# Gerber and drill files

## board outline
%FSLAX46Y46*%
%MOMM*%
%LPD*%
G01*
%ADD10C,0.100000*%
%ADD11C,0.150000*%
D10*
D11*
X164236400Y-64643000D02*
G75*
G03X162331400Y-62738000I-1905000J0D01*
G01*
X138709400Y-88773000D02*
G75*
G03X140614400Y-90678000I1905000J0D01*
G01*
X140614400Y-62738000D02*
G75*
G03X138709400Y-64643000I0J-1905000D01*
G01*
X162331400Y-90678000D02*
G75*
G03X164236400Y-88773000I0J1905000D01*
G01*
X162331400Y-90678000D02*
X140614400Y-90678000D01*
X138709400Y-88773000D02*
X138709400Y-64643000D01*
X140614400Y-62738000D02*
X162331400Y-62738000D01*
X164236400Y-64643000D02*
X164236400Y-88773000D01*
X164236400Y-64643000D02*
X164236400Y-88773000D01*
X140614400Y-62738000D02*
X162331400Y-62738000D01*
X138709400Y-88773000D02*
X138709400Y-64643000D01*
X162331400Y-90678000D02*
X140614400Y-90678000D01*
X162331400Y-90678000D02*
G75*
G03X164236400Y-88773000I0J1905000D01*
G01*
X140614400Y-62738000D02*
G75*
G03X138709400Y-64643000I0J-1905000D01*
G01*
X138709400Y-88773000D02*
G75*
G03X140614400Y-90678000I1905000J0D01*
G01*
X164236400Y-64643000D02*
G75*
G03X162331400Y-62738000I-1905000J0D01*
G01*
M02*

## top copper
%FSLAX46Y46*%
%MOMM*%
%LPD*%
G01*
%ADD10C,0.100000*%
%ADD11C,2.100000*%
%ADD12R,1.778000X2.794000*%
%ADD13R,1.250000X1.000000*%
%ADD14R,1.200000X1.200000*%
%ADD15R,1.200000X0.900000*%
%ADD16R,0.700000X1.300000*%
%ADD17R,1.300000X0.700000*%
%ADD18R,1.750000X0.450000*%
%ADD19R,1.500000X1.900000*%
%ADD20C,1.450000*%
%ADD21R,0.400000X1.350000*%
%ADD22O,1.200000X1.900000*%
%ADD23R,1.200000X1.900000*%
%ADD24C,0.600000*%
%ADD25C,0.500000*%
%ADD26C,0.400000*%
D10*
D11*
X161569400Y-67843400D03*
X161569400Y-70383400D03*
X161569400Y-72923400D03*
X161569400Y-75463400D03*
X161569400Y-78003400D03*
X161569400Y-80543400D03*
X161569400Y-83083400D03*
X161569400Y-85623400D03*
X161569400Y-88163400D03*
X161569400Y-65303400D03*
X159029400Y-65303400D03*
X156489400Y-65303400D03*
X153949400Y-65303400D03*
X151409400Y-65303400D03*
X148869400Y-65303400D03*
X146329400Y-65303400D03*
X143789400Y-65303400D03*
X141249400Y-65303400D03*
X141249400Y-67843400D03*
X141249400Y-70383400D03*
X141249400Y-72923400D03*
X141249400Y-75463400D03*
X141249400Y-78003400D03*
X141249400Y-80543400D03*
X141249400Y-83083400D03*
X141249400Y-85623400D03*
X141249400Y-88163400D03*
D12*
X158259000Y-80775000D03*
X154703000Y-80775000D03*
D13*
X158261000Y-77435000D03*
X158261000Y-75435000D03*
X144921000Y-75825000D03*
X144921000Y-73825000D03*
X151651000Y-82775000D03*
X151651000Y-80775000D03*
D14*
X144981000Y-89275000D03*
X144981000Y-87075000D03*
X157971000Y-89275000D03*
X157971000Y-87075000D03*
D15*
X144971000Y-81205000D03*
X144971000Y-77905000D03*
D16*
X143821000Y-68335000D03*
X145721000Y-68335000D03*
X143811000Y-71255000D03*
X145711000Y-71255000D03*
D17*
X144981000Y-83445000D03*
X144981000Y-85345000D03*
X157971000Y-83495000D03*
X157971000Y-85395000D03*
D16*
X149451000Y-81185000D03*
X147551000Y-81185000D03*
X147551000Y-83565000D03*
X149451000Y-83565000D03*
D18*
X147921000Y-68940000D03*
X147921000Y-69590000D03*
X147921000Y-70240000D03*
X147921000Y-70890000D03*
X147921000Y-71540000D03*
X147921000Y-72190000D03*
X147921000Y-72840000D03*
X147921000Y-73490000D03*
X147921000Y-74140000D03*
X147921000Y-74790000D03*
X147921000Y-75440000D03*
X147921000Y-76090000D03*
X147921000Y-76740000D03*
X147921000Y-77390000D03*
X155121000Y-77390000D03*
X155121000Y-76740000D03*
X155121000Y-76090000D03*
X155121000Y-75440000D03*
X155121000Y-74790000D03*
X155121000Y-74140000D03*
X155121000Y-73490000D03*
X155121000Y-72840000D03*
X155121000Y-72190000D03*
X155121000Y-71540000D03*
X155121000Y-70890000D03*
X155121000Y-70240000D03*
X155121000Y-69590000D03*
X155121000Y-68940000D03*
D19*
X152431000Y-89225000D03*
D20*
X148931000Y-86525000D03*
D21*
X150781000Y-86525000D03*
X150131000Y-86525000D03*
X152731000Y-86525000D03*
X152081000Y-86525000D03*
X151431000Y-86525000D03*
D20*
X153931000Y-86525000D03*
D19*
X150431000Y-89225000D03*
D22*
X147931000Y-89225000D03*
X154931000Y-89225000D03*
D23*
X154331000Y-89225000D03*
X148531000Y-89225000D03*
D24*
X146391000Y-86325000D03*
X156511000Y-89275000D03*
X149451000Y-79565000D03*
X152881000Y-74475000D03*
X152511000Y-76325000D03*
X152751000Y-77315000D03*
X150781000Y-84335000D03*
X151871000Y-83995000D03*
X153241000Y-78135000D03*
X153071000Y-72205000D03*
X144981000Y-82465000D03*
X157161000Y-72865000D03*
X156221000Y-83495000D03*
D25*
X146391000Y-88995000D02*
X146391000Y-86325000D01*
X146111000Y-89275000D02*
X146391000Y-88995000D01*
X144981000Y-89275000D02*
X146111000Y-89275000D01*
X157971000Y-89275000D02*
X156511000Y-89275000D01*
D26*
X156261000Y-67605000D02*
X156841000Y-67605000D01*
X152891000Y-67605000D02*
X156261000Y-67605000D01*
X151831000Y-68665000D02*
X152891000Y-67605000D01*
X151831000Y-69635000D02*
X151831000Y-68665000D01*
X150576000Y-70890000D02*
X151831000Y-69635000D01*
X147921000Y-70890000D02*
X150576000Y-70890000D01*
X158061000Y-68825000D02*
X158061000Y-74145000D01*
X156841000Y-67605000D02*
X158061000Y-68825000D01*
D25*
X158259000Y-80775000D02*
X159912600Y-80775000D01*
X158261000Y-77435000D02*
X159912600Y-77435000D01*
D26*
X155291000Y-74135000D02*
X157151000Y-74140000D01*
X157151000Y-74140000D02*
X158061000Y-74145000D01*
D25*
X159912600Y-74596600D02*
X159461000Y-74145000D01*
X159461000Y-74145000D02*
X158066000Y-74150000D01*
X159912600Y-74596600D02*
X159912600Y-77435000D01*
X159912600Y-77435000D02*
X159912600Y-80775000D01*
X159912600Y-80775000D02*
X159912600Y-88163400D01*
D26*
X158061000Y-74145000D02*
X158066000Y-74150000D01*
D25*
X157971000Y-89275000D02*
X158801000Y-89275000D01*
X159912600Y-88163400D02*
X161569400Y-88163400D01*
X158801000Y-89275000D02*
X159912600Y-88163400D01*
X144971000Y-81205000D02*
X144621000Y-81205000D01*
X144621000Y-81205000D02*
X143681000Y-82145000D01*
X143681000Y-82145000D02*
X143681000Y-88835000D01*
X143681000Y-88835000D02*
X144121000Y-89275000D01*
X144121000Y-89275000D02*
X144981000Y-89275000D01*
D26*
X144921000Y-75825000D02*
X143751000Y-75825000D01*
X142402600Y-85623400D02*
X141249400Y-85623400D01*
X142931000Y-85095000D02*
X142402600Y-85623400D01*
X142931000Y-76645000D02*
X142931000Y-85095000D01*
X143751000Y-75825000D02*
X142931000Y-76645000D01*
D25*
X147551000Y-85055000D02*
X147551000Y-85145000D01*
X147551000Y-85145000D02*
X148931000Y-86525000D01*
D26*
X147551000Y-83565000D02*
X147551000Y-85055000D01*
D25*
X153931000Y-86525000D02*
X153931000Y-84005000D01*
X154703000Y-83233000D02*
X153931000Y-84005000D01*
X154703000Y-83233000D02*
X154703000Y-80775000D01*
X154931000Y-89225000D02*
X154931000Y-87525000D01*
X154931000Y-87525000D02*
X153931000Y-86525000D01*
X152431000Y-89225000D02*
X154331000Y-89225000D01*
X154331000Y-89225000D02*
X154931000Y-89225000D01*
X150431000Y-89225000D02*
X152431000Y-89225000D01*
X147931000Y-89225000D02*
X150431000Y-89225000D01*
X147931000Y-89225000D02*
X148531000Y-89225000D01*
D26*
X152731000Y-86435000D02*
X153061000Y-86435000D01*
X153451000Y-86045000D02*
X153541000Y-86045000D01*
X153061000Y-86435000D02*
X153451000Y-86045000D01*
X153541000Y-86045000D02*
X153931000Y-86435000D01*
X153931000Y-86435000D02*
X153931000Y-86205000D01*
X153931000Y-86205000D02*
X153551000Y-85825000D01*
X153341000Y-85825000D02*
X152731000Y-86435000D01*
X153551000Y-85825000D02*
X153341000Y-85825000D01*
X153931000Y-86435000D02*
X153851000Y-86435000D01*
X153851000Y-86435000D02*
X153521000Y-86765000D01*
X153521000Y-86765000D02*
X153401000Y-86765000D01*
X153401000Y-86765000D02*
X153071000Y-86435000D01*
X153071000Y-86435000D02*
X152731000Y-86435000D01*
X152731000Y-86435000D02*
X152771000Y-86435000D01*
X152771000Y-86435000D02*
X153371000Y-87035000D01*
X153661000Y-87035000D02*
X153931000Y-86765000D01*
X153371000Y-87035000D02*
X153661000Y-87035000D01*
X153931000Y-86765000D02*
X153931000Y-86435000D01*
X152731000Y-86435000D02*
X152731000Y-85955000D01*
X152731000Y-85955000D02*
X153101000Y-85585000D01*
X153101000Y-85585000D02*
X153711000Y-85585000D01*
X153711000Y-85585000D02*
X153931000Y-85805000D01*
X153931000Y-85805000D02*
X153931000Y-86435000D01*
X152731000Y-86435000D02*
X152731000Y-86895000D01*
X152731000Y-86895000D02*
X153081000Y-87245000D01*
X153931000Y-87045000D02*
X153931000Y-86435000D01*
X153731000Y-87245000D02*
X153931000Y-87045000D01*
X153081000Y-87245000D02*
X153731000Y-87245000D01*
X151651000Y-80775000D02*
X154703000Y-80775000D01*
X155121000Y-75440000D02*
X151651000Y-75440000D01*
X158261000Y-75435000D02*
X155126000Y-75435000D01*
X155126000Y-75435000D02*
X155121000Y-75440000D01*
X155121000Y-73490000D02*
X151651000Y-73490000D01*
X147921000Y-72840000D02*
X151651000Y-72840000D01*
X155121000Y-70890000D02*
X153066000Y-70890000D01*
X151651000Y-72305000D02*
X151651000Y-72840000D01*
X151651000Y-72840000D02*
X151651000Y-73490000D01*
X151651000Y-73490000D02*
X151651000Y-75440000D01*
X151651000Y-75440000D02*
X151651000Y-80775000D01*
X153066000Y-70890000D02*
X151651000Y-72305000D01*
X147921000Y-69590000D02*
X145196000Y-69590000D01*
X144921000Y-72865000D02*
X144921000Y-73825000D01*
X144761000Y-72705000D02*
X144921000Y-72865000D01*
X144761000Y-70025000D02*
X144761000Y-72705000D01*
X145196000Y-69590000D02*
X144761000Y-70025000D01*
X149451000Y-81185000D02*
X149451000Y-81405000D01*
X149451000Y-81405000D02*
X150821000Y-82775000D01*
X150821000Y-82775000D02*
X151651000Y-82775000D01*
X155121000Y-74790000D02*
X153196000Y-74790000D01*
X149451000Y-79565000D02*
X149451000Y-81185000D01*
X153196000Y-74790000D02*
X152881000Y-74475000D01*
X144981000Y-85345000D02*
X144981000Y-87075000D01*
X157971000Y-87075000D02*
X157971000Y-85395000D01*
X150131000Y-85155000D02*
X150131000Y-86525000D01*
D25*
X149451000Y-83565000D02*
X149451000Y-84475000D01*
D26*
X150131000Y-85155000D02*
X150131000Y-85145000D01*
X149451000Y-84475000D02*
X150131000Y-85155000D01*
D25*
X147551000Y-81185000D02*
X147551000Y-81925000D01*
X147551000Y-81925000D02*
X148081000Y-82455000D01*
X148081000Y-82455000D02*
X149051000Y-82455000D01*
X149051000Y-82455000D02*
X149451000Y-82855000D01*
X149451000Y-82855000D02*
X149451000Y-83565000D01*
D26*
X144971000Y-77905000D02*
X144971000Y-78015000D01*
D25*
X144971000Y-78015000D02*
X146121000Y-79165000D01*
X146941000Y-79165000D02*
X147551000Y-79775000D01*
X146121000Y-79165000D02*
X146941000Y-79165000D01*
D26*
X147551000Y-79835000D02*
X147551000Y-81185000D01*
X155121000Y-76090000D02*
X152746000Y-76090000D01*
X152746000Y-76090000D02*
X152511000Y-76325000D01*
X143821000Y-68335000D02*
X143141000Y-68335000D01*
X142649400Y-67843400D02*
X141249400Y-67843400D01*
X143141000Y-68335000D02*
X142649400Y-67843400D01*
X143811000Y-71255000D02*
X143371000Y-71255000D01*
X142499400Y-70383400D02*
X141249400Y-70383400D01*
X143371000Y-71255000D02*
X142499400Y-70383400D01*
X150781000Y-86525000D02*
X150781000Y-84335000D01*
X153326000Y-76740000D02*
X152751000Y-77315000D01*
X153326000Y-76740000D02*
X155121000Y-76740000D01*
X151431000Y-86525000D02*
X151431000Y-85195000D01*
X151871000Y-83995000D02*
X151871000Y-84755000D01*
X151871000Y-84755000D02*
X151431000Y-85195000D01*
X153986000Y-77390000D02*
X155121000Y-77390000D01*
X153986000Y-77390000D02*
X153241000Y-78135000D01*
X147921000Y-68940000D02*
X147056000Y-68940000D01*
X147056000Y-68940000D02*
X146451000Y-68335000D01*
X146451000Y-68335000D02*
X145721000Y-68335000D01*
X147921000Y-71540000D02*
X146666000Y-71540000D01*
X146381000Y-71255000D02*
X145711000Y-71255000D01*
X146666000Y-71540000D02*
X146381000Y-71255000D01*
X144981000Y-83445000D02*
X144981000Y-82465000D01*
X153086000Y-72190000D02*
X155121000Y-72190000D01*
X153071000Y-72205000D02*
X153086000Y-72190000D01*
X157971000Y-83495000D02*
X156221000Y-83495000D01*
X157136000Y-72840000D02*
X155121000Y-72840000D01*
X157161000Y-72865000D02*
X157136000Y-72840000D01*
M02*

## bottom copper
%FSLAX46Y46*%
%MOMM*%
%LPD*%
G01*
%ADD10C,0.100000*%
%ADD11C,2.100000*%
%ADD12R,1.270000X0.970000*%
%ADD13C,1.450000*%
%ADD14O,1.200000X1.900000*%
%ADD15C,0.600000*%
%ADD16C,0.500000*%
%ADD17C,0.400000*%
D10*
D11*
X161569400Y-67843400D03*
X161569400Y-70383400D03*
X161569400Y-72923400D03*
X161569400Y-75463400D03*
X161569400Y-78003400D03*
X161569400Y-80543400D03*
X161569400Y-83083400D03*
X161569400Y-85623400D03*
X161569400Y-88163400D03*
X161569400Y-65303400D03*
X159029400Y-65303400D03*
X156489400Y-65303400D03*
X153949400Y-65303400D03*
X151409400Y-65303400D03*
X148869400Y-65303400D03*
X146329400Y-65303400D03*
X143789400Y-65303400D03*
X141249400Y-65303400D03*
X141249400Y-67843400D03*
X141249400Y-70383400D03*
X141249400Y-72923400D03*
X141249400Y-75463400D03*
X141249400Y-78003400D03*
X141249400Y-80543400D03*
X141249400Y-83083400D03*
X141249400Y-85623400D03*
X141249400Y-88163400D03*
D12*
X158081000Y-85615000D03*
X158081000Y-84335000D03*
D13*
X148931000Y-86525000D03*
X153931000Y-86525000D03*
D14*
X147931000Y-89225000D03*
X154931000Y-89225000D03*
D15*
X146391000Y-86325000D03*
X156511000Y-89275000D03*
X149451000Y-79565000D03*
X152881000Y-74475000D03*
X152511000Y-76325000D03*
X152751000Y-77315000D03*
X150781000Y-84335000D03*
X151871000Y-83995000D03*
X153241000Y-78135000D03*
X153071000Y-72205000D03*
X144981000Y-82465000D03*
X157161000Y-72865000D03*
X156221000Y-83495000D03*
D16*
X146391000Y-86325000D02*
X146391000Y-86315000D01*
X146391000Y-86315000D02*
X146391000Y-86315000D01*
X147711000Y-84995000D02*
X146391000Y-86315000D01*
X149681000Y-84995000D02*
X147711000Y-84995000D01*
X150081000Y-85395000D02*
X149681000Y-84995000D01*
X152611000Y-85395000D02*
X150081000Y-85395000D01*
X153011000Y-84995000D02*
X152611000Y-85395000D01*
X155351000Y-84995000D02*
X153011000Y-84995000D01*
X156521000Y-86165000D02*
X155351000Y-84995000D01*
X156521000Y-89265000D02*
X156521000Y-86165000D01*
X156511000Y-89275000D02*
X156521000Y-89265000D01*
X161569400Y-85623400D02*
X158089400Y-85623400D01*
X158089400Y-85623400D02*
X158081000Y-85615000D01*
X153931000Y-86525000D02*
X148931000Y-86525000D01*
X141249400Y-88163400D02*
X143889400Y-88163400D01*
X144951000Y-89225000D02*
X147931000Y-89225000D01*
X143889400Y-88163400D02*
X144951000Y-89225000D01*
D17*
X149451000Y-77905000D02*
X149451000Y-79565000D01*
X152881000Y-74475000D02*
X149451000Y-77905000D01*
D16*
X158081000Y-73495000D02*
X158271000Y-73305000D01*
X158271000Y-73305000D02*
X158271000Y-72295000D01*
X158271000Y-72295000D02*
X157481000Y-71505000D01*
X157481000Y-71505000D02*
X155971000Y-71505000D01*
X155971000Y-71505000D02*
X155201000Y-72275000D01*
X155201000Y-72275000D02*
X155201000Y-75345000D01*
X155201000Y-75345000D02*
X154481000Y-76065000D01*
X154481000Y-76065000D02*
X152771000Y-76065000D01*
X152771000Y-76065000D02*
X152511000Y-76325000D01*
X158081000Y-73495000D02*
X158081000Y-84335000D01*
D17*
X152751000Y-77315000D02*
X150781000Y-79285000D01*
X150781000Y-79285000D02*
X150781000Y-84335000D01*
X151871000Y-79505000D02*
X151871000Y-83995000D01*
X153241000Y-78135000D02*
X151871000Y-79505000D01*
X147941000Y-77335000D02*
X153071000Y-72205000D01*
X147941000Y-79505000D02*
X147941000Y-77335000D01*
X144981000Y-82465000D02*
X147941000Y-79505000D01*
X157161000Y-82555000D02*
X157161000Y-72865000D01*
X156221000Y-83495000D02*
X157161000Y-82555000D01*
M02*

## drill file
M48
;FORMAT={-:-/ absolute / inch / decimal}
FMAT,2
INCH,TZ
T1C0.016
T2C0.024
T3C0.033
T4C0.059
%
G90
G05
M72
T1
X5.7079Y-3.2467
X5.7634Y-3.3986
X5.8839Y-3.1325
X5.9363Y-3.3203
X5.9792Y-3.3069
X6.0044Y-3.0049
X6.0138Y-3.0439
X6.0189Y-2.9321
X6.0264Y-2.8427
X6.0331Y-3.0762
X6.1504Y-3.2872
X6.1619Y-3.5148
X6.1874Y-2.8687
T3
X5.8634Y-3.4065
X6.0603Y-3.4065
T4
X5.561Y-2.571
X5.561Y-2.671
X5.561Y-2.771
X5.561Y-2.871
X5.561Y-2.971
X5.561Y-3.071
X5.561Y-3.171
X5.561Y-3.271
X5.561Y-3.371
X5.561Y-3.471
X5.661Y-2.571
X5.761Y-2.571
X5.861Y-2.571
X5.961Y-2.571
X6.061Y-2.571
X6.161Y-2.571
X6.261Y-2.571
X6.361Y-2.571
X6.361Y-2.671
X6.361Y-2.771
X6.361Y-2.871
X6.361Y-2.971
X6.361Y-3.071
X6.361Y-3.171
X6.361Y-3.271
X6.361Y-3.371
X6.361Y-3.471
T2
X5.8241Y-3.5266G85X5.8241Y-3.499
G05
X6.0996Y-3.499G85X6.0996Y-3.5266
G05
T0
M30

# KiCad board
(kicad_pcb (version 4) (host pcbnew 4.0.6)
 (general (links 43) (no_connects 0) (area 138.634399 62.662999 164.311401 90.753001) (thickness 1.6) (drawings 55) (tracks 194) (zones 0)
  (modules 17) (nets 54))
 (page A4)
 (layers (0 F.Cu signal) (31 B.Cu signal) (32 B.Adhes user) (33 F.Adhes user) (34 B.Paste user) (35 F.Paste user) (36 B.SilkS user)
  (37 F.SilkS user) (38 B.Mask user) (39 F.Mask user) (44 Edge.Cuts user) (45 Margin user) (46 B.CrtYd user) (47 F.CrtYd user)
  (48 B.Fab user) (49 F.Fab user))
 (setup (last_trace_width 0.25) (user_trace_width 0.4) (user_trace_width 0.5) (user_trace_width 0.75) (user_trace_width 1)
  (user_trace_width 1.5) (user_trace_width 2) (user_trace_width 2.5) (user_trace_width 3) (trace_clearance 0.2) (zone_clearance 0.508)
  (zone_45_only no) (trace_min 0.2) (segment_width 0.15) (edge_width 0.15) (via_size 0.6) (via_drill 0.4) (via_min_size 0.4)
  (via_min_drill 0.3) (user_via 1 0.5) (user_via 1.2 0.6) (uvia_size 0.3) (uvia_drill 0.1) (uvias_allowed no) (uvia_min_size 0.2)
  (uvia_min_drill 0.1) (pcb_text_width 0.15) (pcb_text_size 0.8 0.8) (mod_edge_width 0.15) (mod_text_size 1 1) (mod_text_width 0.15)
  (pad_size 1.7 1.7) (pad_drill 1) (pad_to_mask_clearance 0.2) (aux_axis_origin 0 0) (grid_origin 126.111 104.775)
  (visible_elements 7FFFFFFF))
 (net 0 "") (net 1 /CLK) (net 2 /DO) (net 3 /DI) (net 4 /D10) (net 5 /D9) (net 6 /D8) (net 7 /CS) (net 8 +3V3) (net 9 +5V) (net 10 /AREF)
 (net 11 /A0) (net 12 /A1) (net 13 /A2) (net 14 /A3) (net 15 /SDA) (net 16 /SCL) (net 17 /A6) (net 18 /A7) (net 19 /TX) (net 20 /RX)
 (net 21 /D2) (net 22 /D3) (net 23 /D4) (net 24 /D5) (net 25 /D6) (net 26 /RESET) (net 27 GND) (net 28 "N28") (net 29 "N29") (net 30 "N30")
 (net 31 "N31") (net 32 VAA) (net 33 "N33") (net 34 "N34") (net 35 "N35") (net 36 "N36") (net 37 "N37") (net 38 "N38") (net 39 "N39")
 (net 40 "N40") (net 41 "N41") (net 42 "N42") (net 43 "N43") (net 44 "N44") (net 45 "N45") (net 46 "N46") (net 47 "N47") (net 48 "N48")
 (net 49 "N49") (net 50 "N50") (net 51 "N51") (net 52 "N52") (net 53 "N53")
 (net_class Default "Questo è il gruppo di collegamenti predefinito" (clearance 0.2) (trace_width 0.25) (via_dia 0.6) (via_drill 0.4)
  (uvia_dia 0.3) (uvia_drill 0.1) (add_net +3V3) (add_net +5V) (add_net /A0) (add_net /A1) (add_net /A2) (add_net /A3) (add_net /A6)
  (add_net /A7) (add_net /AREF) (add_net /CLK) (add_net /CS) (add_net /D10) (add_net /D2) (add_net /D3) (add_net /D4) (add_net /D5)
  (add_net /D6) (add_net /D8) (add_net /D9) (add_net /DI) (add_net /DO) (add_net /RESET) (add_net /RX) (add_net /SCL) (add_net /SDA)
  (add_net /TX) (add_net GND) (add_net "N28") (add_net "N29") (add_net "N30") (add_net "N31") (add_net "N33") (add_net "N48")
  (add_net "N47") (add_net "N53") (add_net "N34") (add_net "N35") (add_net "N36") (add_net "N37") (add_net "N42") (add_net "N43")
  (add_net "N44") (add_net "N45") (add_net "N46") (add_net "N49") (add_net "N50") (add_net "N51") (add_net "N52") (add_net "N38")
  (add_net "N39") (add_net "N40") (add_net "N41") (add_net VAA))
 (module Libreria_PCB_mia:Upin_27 (layer B.Cu) (at 161.5694 88.1634 180)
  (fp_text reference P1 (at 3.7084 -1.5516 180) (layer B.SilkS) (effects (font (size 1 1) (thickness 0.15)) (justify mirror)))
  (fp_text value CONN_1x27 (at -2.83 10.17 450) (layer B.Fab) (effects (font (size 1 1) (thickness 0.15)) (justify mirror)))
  (pad 9 thru_hole circle (at 0 20.32 180) (size 2.1 2.1) (drill 1.5) (layers *.Cu *.Mask) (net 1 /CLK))
  (pad 8 thru_hole circle (at 0 17.78 180) (size 2.1 2.1) (drill 1.5) (layers *.Cu *.Mask) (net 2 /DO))
  (pad 7 thru_hole circle (at 0 15.24 180) (size 2.1 2.1) (drill 1.5) (layers *.Cu *.Mask) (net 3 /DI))
  (pad 6 thru_hole circle (at 0 12.7 180) (size 2.1 2.1) (drill 1.5) (layers *.Cu *.Mask) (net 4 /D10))
  (pad 5 thru_hole circle (at 0 10.16 180) (size 2.1 2.1) (drill 1.5) (layers *.Cu *.Mask) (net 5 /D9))
  (pad 4 thru_hole circle (at 0 7.62 180) (size 2.1 2.1) (drill 1.5) (layers *.Cu *.Mask) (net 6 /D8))
  (pad 3 thru_hole circle (at 0 5.08 180) (size 2.1 2.1) (drill 1.5) (layers *.Cu *.Mask) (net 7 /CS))
  (pad 2 thru_hole circle (at 0 2.54 180) (size 2.1 2.1) (drill 1.5) (layers *.Cu *.Mask) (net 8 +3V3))
  (pad 1 thru_hole circle (at 0 0 180) (size 2.1 2.1) (drill 1.5) (layers *.Cu *.Mask) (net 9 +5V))
  (pad 10 thru_hole circle (at 0 22.86 180) (size 2.1 2.1) (drill 1.5) (layers *.Cu *.Mask) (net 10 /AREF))
  (pad 11 thru_hole circle (at 2.54 22.86 180) (size 2.1 2.1) (drill 1.5) (layers *.Cu *.Mask) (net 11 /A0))
  (pad 12 thru_hole circle (at 5.08 22.86 180) (size 2.1 2.1) (drill 1.5) (layers *.Cu *.Mask) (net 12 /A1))
  (pad 13 thru_hole circle (at 7.62 22.86 180) (size 2.1 2.1) (drill 1.5) (layers *.Cu *.Mask) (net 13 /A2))
  (pad 14 thru_hole circle (at 10.16 22.86 180) (size 2.1 2.1) (drill 1.5) (layers *.Cu *.Mask) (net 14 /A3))
  (pad 15 thru_hole circle (at 12.7 22.86 180) (size 2.1 2.1) (drill 1.5) (layers *.Cu *.Mask) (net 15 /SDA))
  (pad 16 thru_hole circle (at 15.24 22.86 180) (size 2.1 2.1) (drill 1.5) (layers *.Cu *.Mask) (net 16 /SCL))
  (pad 17 thru_hole circle (at 17.78 22.86 180) (size 2.1 2.1) (drill 1.5) (layers *.Cu *.Mask) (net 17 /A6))
  (pad 18 thru_hole circle (at 20.32 22.86 180) (size 2.1 2.1) (drill 1.5) (layers *.Cu *.Mask) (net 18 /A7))
  (pad 19 thru_hole circle (at 20.32 20.32 180) (size 2.1 2.1) (drill 1.5) (layers *.Cu *.Mask) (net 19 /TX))
  (pad 20 thru_hole circle (at 20.32 17.78 180) (size 2.1 2.1) (drill 1.5) (layers *.Cu *.Mask) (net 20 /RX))
  (pad 21 thru_hole circle (at 20.32 15.24 180) (size 2.1 2.1) (drill 1.5) (layers *.Cu *.Mask) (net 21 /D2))
  (pad 22 thru_hole circle (at 20.32 12.7 180) (size 2.1 2.1) (drill 1.5) (layers *.Cu *.Mask) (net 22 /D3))
  (pad 23 thru_hole circle (at 20.32 10.16 180) (size 2.1 2.1) (drill 1.5) (layers *.Cu *.Mask) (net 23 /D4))
  (pad 24 thru_hole circle (at 20.32 7.62 180) (size 2.1 2.1) (drill 1.5) (layers *.Cu *.Mask) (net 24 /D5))
  (pad 25 thru_hole circle (at 20.32 5.08 180) (size 2.1 2.1) (drill 1.5) (layers *.Cu *.Mask) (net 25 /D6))
  (pad 26 thru_hole circle (at 20.32 2.54 180) (size 2.1 2.1) (drill 1.5) (layers *.Cu *.Mask) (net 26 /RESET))
  (pad 27 thru_hole circle (at 20.32 0 180) (size 2.1 2.1) (drill 1.5) (layers *.Cu *.Mask) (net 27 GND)))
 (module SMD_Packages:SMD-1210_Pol (layer F.Cu) (at 156.481 80.775 180)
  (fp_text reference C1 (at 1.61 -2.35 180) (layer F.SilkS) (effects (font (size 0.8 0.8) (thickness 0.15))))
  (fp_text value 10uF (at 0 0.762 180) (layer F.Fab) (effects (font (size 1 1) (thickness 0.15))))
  (pad 1 smd rect (at -1.778 0 180) (size 1.778 2.794) (layers F.Cu F.Paste F.Mask) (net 9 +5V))
  (pad 2 smd rect (at 1.778 0 180) (size 1.778 2.794) (layers F.Cu F.Paste F.Mask) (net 27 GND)))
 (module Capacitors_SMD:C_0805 (layer F.Cu) (at 158.261 76.435 90)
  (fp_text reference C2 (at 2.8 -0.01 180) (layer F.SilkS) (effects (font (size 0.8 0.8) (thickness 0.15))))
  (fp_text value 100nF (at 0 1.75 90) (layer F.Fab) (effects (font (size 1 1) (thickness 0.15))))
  (pad 1 smd rect (at -1 0 90) (size 1 1.25) (layers F.Cu F.Paste F.Mask) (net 9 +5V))
  (pad 2 smd rect (at 1 0 90) (size 1 1.25) (layers F.Cu F.Paste F.Mask) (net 27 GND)))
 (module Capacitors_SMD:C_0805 (layer F.Cu) (at 144.921 74.825 90)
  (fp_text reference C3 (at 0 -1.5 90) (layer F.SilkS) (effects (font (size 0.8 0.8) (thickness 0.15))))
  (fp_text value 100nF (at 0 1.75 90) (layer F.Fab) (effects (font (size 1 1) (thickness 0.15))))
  (pad 1 smd rect (at -1 0 90) (size 1 1.25) (layers F.Cu F.Paste F.Mask) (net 26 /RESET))
  (pad 2 smd rect (at 1 0 90) (size 1 1.25) (layers F.Cu F.Paste F.Mask) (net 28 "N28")))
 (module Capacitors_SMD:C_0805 (layer F.Cu) (at 151.651 81.775 90)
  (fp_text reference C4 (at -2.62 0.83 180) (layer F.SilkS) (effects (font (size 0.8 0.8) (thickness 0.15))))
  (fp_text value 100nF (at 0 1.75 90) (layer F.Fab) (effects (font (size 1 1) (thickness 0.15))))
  (pad 1 smd rect (at -1 0 90) (size 1 1.25) (layers F.Cu F.Paste F.Mask) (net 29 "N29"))
  (pad 2 smd rect (at 1 0 90) (size 1 1.25) (layers F.Cu F.Paste F.Mask) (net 27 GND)))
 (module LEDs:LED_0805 (layer F.Cu) (at 144.981 88.175 270)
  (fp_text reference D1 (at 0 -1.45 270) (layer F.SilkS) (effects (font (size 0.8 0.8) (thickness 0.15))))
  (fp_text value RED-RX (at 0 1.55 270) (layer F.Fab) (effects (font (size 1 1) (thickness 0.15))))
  (pad 2 smd rect (at 1.1 0 90) (size 1.2 1.2) (layers F.Cu F.Paste F.Mask) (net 9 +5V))
  (pad 1 smd rect (at -1.1 0 90) (size 1.2 1.2) (layers F.Cu F.Paste F.Mask) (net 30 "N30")))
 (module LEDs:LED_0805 (layer F.Cu) (at 157.971 88.175 270)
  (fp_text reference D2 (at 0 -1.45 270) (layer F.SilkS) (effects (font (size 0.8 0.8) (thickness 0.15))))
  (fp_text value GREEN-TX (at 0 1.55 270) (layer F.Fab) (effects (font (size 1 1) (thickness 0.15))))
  (pad 2 smd rect (at 1.1 0 90) (size 1.2 1.2) (layers F.Cu F.Paste F.Mask) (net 9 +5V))
  (pad 1 smd rect (at -1.1 0 90) (size 1.2 1.2) (layers F.Cu F.Paste F.Mask) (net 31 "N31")))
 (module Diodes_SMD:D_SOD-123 (layer F.Cu) (at 144.971 79.555 90)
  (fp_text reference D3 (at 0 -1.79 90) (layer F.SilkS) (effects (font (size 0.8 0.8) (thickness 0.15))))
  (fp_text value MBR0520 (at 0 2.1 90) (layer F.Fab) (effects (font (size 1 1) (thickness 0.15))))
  (pad 1 smd rect (at -1.65 0 90) (size 0.9 1.2) (layers F.Cu F.Paste F.Mask) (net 9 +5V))
  (pad 2 smd rect (at 1.65 0 90) (size 0.9 1.2) (layers F.Cu F.Paste F.Mask) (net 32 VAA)))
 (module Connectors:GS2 (layer B.Cu) (at 158.081 84.975)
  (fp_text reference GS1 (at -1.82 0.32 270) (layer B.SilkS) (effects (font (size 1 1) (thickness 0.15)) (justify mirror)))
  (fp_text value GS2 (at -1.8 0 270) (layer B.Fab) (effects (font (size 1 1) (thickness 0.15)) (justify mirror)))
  (pad 1 smd rect (at 0 0.64) (size 1.27 0.97) (layers B.Cu B.Paste B.Mask) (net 8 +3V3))
  (pad 2 smd rect (at 0 -0.64) (size 1.27 0.97) (layers B.Cu B.Paste B.Mask) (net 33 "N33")))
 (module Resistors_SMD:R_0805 (layer F.Cu) (at 144.771 68.335)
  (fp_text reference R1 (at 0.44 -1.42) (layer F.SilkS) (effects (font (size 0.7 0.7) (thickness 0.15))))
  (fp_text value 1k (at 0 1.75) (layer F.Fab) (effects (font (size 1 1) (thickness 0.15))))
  (pad 1 smd rect (at -0.95 0) (size 0.7 1.3) (layers F.Cu F.Paste F.Mask) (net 19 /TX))
  (pad 2 smd rect (at 0.95 0) (size 0.7 1.3) (layers F.Cu F.Paste F.Mask) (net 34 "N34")))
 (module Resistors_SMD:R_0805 (layer F.Cu) (at 144.761 71.255)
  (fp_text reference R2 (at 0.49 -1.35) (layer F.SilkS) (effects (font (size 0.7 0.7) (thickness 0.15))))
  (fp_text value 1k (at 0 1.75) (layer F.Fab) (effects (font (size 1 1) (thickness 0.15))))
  (pad 1 smd rect (at -0.95 0) (size 0.7 1.3) (layers F.Cu F.Paste F.Mask) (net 20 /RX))
  (pad 2 smd rect (at 0.95 0) (size 0.7 1.3) (layers F.Cu F.Paste F.Mask) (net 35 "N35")))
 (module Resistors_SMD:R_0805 (layer F.Cu) (at 144.981 84.395 270)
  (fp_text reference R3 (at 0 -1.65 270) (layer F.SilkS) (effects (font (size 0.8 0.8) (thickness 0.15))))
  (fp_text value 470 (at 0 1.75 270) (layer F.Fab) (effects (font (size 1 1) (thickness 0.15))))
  (pad 1 smd rect (at -0.95 0 270) (size 0.7 1.3) (layers F.Cu F.Paste F.Mask) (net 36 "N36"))
  (pad 2 smd rect (at 0.95 0 270) (size 0.7 1.3) (layers F.Cu F.Paste F.Mask) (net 30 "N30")))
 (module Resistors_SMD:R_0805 (layer F.Cu) (at 157.971 84.445 270)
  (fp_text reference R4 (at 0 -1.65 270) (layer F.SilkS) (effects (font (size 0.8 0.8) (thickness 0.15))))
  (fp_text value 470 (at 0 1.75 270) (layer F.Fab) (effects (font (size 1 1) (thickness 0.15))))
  (pad 1 smd rect (at -0.95 0 270) (size 0.7 1.3) (layers F.Cu F.Paste F.Mask) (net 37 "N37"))
  (pad 2 smd rect (at 0.95 0 270) (size 0.7 1.3) (layers F.Cu F.Paste F.Mask) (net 31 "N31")))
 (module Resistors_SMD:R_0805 (layer F.Cu) (at 148.501 81.185 180)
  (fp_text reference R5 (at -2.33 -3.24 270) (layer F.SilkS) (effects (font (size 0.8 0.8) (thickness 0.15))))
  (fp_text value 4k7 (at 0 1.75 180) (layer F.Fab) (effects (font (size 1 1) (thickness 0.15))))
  (pad 1 smd rect (at -0.95 0 180) (size 0.7 1.3) (layers F.Cu F.Paste F.Mask) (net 29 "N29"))
  (pad 2 smd rect (at 0.95 0 180) (size 0.7 1.3) (layers F.Cu F.Paste F.Mask) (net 32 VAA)))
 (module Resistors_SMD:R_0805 (layer F.Cu) (at 148.501 83.565)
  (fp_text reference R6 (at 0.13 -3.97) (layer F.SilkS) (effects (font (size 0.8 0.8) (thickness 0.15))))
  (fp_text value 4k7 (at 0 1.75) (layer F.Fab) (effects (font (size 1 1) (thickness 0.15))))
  (pad 1 smd rect (at -0.95 0) (size 0.7 1.3) (layers F.Cu F.Paste F.Mask) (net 27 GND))
  (pad 2 smd rect (at 0.95 0) (size 0.7 1.3) (layers F.Cu F.Paste F.Mask) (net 32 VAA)))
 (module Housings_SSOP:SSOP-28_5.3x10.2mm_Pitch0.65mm (layer F.Cu) (at 151.521 73.165)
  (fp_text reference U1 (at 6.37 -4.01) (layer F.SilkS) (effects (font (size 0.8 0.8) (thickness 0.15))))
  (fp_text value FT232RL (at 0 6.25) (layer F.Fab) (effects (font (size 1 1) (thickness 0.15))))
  (pad 1 smd rect (at -3.6 -4.225) (size 1.75 0.45) (layers F.Cu F.Paste F.Mask) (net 34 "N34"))
  (pad 2 smd rect (at -3.6 -3.575) (size 1.75 0.45) (layers F.Cu F.Paste F.Mask) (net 28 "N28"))
  (pad 3 smd rect (at -3.6 -2.925) (size 1.75 0.45) (layers F.Cu F.Paste F.Mask) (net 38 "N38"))
  (pad 4 smd rect (at -3.6 -2.275) (size 1.75 0.45) (layers F.Cu F.Paste F.Mask) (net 9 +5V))
  (pad 5 smd rect (at -3.6 -1.625) (size 1.75 0.45) (layers F.Cu F.Paste F.Mask) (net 35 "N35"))
  (pad 6 smd rect (at -3.6 -0.975) (size 1.75 0.45) (layers F.Cu F.Paste F.Mask) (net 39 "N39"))
  (pad 7 smd rect (at -3.6 -0.325) (size 1.75 0.45) (layers F.Cu F.Paste F.Mask) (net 27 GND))
  (pad 8 smd rect (at -3.6 0.325) (size 1.75 0.45) (layers F.Cu F.Paste F.Mask) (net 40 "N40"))
  (pad 9 smd rect (at -3.6 0.975) (size 1.75 0.45) (layers F.Cu F.Paste F.Mask) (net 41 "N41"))
  (pad 10 smd rect (at -3.6 1.625) (size 1.75 0.45) (layers F.Cu F.Paste F.Mask) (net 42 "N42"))
  (pad 11 smd rect (at -3.6 2.275) (size 1.75 0.45) (layers F.Cu F.Paste F.Mask) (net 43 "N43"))
  (pad 12 smd rect (at -3.6 2.925) (size 1.75 0.45) (layers F.Cu F.Paste F.Mask) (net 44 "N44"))
  (pad 13 smd rect (at -3.6 3.575) (size 1.75 0.45) (layers F.Cu F.Paste F.Mask) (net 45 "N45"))
  (pad 14 smd rect (at -3.6 4.225) (size 1.75 0.45) (layers F.Cu F.Paste F.Mask) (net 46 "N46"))
  (pad 15 smd rect (at 3.6 4.225) (size 1.75 0.45) (layers F.Cu F.Paste F.Mask) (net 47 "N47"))
  (pad 16 smd rect (at 3.6 3.575) (size 1.75 0.45) (layers F.Cu F.Paste F.Mask) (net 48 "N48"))
  (pad 17 smd rect (at 3.6 2.925) (size 1.75 0.45) (layers F.Cu F.Paste F.Mask) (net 33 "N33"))
  (pad 18 smd rect (at 3.6 2.275) (size 1.75 0.45) (layers F.Cu F.Paste F.Mask) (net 27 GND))
  (pad 19 smd rect (at 3.6 1.625) (size 1.75 0.45) (layers F.Cu F.Paste F.Mask) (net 29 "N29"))
  (pad 20 smd rect (at 3.6 0.975) (size 1.75 0.45) (layers F.Cu F.Paste F.Mask) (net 9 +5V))
  (pad 21 smd rect (at 3.6 0.325) (size 1.75 0.45) (layers F.Cu F.Paste F.Mask) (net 27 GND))
  (pad 22 smd rect (at 3.6 -0.325) (size 1.75 0.45) (layers F.Cu F.Paste F.Mask) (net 37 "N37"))
  (pad 23 smd rect (at 3.6 -0.975) (size 1.75 0.45) (layers F.Cu F.Paste F.Mask) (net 36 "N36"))
  (pad 24 smd rect (at 3.6 -1.625) (size 1.75 0.45) (layers F.Cu F.Paste F.Mask) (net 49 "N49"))
  (pad 25 smd rect (at 3.6 -2.275) (size 1.75 0.45) (layers F.Cu F.Paste F.Mask) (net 27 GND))
  (pad 26 smd rect (at 3.6 -2.925) (size 1.75 0.45) (layers F.Cu F.Paste F.Mask) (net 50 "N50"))
  (pad 27 smd rect (at 3.6 -3.575) (size 1.75 0.45) (layers F.Cu F.Paste F.Mask) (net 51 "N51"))
  (pad 28 smd rect (at 3.6 -4.225) (size 1.75 0.45) (layers F.Cu F.Paste F.Mask) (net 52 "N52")))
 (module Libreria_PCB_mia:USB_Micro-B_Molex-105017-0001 (layer F.Cu) (at 151.431 88.875)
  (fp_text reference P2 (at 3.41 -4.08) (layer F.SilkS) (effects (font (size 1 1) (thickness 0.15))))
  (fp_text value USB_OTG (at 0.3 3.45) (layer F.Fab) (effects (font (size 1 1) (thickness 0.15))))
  (pad 6 smd rect (at 1 0.35) (size 1.5 1.9) (layers F.Cu F.Paste F.Mask) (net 27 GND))
  (pad 6 thru_hole circle (at -2.5 -2.35) (size 1.45 1.45) (drill 0.85) (layers *.Cu *.Mask) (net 27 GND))
  (pad 2 smd rect (at -0.65 -2.35) (size 0.4 1.35) (layers F.Cu F.Paste F.Mask) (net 48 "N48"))
  (pad 1 smd rect (at -1.3 -2.35) (size 0.4 1.35) (layers F.Cu F.Paste F.Mask) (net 32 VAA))
  (pad 5 smd rect (at 1.3 -2.35) (size 0.4 1.35) (layers F.Cu F.Paste F.Mask) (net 27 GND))
  (pad 4 smd rect (at 0.65 -2.35) (size 0.4 1.35) (layers F.Cu F.Paste F.Mask) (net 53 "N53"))
  (pad 3 smd rect (at 0 -2.35) (size 0.4 1.35) (layers F.Cu F.Paste F.Mask) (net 47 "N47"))
  (pad 6 thru_hole circle (at 2.5 -2.35) (size 1.45 1.45) (drill 0.85) (layers *.Cu *.Mask) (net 27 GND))
  (pad 6 smd rect (at -1 0.35) (size 1.5 1.9) (layers F.Cu F.Paste F.Mask) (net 27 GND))
  (pad 6 thru_hole oval (at -3.5 0.35 180) (size 1.2 1.9) (drill oval 0.6 1.3) (layers *.Cu *.Mask) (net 27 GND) (zone_connect 0))
  (pad 6 thru_hole oval (at 3.5 0.35) (size 1.2 1.9) (drill oval 0.6 1.3) (layers *.Cu *.Mask) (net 27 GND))
  (pad 6 smd rect (at 2.9 0.35) (size 1.2 1.9) (layers F.Cu F.Mask) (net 27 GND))
  (pad 6 smd rect (at -2.9 0.35) (size 1.2 1.9) (layers F.Cu F.Mask) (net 27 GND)))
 (gr_arc (start 162.3314 64.643) (end 162.3314 62.738) (angle 90) (layer Edge.Cuts) (width 0.15))
 (gr_arc (start 140.6144 88.773) (end 140.6144 90.678) (angle 90) (layer Edge.Cuts) (width 0.15))
 (gr_arc (start 140.6144 64.643) (end 138.7094 64.643) (angle 90) (layer Edge.Cuts) (width 0.15))
 (gr_arc (start 162.3314 88.773) (end 164.2364 88.773) (angle 90) (layer Edge.Cuts) (width 0.15))
 (gr_line (start 162.3314 90.678) (end 140.6144 90.678) (angle 90) (layer Edge.Cuts) (width 0.15))
 (gr_line (start 138.7094 88.773) (end 138.7094 64.643) (angle 90) (layer Edge.Cuts) (width 0.15))
 (gr_line (start 140.6144 62.738) (end 162.3314 62.738) (angle 90) (layer Edge.Cuts) (width 0.15))
 (gr_line (start 164.2364 64.643) (end 164.2364 88.773) (angle 90) (layer Edge.Cuts) (width 0.15))
 (gr_line (start 164.2364 64.643) (end 164.2364 88.773) (angle 90) (layer Edge.Cuts) (width 0.15))
 (gr_line (start 140.6144 62.738) (end 162.3314 62.738) (angle 90) (layer Edge.Cuts) (width 0.15))
 (gr_line (start 138.7094 88.773) (end 138.7094 64.643) (angle 90) (layer Edge.Cuts) (width 0.15))
 (gr_line (start 162.3314 90.678) (end 140.6144 90.678) (angle 90) (layer Edge.Cuts) (width 0.15))
 (gr_arc (start 162.3314 88.773) (end 164.2364 88.773) (angle 90) (layer Edge.Cuts) (width 0.15))
 (gr_arc (start 140.6144 64.643) (end 138.7094 64.643) (angle 90) (layer Edge.Cuts) (width 0.15))
 (gr_arc (start 140.6144 88.773) (end 140.6144 90.678) (angle 90) (layer Edge.Cuts) (width 0.15))
 (gr_arc (start 162.3314 64.643) (end 162.3314 62.738) (angle 90) (layer Edge.Cuts) (width 0.15))
 (segment (start 146.391 86.325) (end 146.391 86.315) (width 0.5) (layer B.Cu) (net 9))
 (via (at 146.391 86.325) (size 0.6) (drill 0.4) (layers F.Cu B.Cu) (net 9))
 (segment (start 146.391 88.995) (end 146.391 86.325) (width 0.5) (layer F.Cu) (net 9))
 (segment (start 146.111 89.275) (end 146.391 88.995) (width 0.5) (layer F.Cu) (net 9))
 (segment (start 144.981 89.275) (end 146.111 89.275) (width 0.5) (layer F.Cu) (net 9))
 (segment (start 146.391 86.315) (end 146.391 86.315) (width 0.5) (layer B.Cu) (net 9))
 (segment (start 157.971 89.275) (end 156.511 89.275) (width 0.5) (layer F.Cu) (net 9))
 (segment (start 147.711 84.995) (end 146.391 86.315) (width 0.5) (layer B.Cu) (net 9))
 (segment (start 149.681 84.995) (end 147.711 84.995) (width 0.5) (layer B.Cu) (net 9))
 (segment (start 150.081 85.395) (end 149.681 84.995) (width 0.5) (layer B.Cu) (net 9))
 (segment (start 152.611 85.395) (end 150.081 85.395) (width 0.5) (layer B.Cu) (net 9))
 (segment (start 153.011 84.995) (end 152.611 85.395) (width 0.5) (layer B.Cu) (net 9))
 (segment (start 155.351 84.995) (end 153.011 84.995) (width 0.5) (layer B.Cu) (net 9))
 (segment (start 156.521 86.165) (end 155.351 84.995) (width 0.5) (layer B.Cu) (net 9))
 (segment (start 156.521 89.265) (end 156.521 86.165) (width 0.5) (layer B.Cu) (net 9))
 (segment (start 156.511 89.275) (end 156.521 89.265) (width 0.5) (layer B.Cu) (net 9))
 (via (at 156.511 89.275) (size 0.6) (drill 0.4) (layers F.Cu B.Cu) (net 9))
 (segment (start 156.261 67.605) (end 156.841 67.605) (width 0.4) (layer F.Cu) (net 9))
 (segment (start 152.891 67.605) (end 156.261 67.605) (width 0.4) (layer F.Cu) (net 9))
 (segment (start 151.831 68.665) (end 152.891 67.605) (width 0.4) (layer F.Cu) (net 9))
 (segment (start 151.831 69.635) (end 151.831 68.665) (width 0.4) (layer F.Cu) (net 9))
 (segment (start 150.576 70.89) (end 151.831 69.635) (width 0.4) (layer F.Cu) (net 9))
 (segment (start 147.921 70.89) (end 150.576 70.89) (width 0.4) (layer F.Cu) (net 9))
 (segment (start 158.061 68.825) (end 158.061 74.145) (width 0.4) (layer F.Cu) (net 9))
 (segment (start 156.841 67.605) (end 158.061 68.825) (width 0.4) (layer F.Cu) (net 9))
 (segment (start 158.259 80.775) (end 159.9126 80.775) (width 0.5) (layer F.Cu) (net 9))
 (segment (start 158.261 77.435) (end 159.9126 77.435) (width 0.5) (layer F.Cu) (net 9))
 (segment (start 155.291 74.135) (end 157.151 74.14) (width 0.4) (layer F.Cu) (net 9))
 (segment (start 157.151 74.14) (end 158.061 74.145) (width 0.4) (layer F.Cu) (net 9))
 (segment (start 159.9126 74.5966) (end 159.461 74.145) (width 0.5) (layer F.Cu) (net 9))
 (segment (start 159.461 74.145) (end 158.066 74.15) (width 0.5) (layer F.Cu) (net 9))
 (segment (start 159.9126 74.5966) (end 159.9126 77.435) (width 0.5) (layer F.Cu) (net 9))
 (segment (start 159.9126 77.435) (end 159.9126 80.775) (width 0.5) (layer F.Cu) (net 9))
 (segment (start 159.9126 80.775) (end 159.9126 88.1634) (width 0.5) (layer F.Cu) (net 9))
 (segment (start 158.061 74.145) (end 158.066 74.15) (width 0.4) (layer F.Cu) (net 9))
 (segment (start 157.971 89.275) (end 158.801 89.275) (width 0.5) (layer F.Cu) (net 9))
 (segment (start 159.9126 88.1634) (end 161.5694 88.1634) (width 0.5) (layer F.Cu) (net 9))
 (segment (start 158.801 89.275) (end 159.9126 88.1634) (width 0.5) (layer F.Cu) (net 9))
 (segment (start 144.971 81.205) (end 144.621 81.205) (width 0.5) (layer F.Cu) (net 9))
 (segment (start 144.621 81.205) (end 143.681 82.145) (width 0.5) (layer F.Cu) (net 9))
 (segment (start 143.681 82.145) (end 143.681 88.835) (width 0.5) (layer F.Cu) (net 9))
 (segment (start 143.681 88.835) (end 144.121 89.275) (width 0.5) (layer F.Cu) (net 9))
 (segment (start 144.121 89.275) (end 144.981 89.275) (width 0.5) (layer F.Cu) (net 9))
 (segment (start 161.5694 85.6234) (end 158.0894 85.6234) (width 0.5) (layer B.Cu) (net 8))
 (segment (start 158.0894 85.6234) (end 158.081 85.615) (width 0.5) (layer B.Cu) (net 8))
 (segment (start 144.921 75.825) (end 143.751 75.825) (width 0.4) (layer F.Cu) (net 26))
 (segment (start 142.4026 85.6234) (end 141.2494 85.6234) (width 0.4) (layer F.Cu) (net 26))
 (segment (start 142.931 85.095) (end 142.4026 85.6234) (width 0.4) (layer F.Cu) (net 26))
 (segment (start 142.931 76.645) (end 142.931 85.095) (width 0.4) (layer F.Cu) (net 26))
 (segment (start 143.751 75.825) (end 142.931 76.645) (width 0.4) (layer F.Cu) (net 26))
 (segment (start 153.931 86.525) (end 148.931 86.525) (width 0.5) (layer B.Cu) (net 27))
 (segment (start 147.551 85.055) (end 147.551 85.145) (width 0.5) (layer F.Cu) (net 27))
 (segment (start 147.551 85.145) (end 148.931 86.525) (width 0.5) (layer F.Cu) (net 27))
 (segment (start 147.551 83.565) (end 147.551 85.055) (width 0.4) (layer F.Cu) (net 27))
 (segment (start 153.931 86.525) (end 153.931 84.005) (width 0.5) (layer F.Cu) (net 27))
 (segment (start 154.703 83.233) (end 153.931 84.005) (width 0.5) (layer F.Cu) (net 27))
 (segment (start 154.703 83.233) (end 154.703 80.775) (width 0.5) (layer F.Cu) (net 27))
 (segment (start 154.931 89.225) (end 154.931 87.525) (width 0.5) (layer F.Cu) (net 27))
 (segment (start 154.931 87.525) (end 153.931 86.525) (width 0.5) (layer F.Cu) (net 27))
 (segment (start 152.431 89.225) (end 154.331 89.225) (width 0.5) (layer F.Cu) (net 27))
 (segment (start 154.331 89.225) (end 154.931 89.225) (width 0.5) (layer F.Cu) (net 27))
 (segment (start 150.431 89.225) (end 152.431 89.225) (width 0.5) (layer F.Cu) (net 27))
 (segment (start 147.931 89.225) (end 150.431 89.225) (width 0.5) (layer F.Cu) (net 27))
 (segment (start 147.931 89.225) (end 148.531 89.225) (width 0.5) (layer F.Cu) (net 27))
 (segment (start 141.2494 88.1634) (end 143.8894 88.1634) (width 0.5) (layer B.Cu) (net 27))
 (segment (start 144.951 89.225) (end 147.931 89.225) (width 0.5) (layer B.Cu) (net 27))
 (segment (start 143.8894 88.1634) (end 144.951 89.225) (width 0.5) (layer B.Cu) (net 27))
 (segment (start 152.731 86.435) (end 153.061 86.435) (width 0.4) (layer F.Cu) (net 27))
 (segment (start 153.451 86.045) (end 153.541 86.045) (width 0.4) (layer F.Cu) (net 27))
 (segment (start 153.061 86.435) (end 153.451 86.045) (width 0.4) (layer F.Cu) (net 27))
 (segment (start 153.541 86.045) (end 153.931 86.435) (width 0.4) (layer F.Cu) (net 27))
 (segment (start 153.931 86.435) (end 153.931 86.205) (width 0.4) (layer F.Cu) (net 27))
 (segment (start 153.931 86.205) (end 153.551 85.825) (width 0.4) (layer F.Cu) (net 27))
 (segment (start 153.341 85.825) (end 152.731 86.435) (width 0.4) (layer F.Cu) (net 27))
 (segment (start 153.551 85.825) (end 153.341 85.825) (width 0.4) (layer F.Cu) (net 27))
 (segment (start 153.931 86.435) (end 153.851 86.435) (width 0.4) (layer F.Cu) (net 27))
 (segment (start 153.851 86.435) (end 153.521 86.765) (width 0.4) (layer F.Cu) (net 27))
 (segment (start 153.521 86.765) (end 153.401 86.765) (width 0.4) (layer F.Cu) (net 27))
 (segment (start 153.401 86.765) (end 153.071 86.435) (width 0.4) (layer F.Cu) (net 27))
 (segment (start 153.071 86.435) (end 152.731 86.435) (width 0.4) (layer F.Cu) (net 27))
 (segment (start 152.731 86.435) (end 152.771 86.435) (width 0.4) (layer F.Cu) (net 27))
 (segment (start 152.771 86.435) (end 153.371 87.035) (width 0.4) (layer F.Cu) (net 27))
 (segment (start 153.661 87.035) (end 153.931 86.765) (width 0.4) (layer F.Cu) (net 27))
 (segment (start 153.371 87.035) (end 153.661 87.035) (width 0.4) (layer F.Cu) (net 27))
 (segment (start 153.931 86.765) (end 153.931 86.435) (width 0.4) (layer F.Cu) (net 27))
 (segment (start 152.731 86.435) (end 152.731 85.955) (width 0.4) (layer F.Cu) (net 27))
 (segment (start 152.731 85.955) (end 153.101 85.585) (width 0.4) (layer F.Cu) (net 27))
 (segment (start 153.101 85.585) (end 153.711 85.585) (width 0.4) (layer F.Cu) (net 27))
 (segment (start 153.711 85.585) (end 153.931 85.805) (width 0.4) (layer F.Cu) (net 27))
 (segment (start 153.931 85.805) (end 153.931 86.435) (width 0.4) (layer F.Cu) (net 27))
 (segment (start 152.731 86.435) (end 152.731 86.895) (width 0.4) (layer F.Cu) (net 27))
 (segment (start 152.731 86.895) (end 153.081 87.245) (width 0.4) (layer F.Cu) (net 27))
 (segment (start 153.931 87.045) (end 153.931 86.435) (width 0.4) (layer F.Cu) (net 27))
 (segment (start 153.731 87.245) (end 153.931 87.045) (width 0.4) (layer F.Cu) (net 27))
 (segment (start 153.081 87.245) (end 153.731 87.245) (width 0.4) (layer F.Cu) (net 27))
 (segment (start 151.651 80.775) (end 154.703 80.775) (width 0.4) (layer F.Cu) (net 27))
 (segment (start 155.121 75.44) (end 151.651 75.44) (width 0.4) (layer F.Cu) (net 27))
 (segment (start 158.261 75.435) (end 155.126 75.435) (width 0.4) (layer F.Cu) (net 27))
 (segment (start 155.126 75.435) (end 155.121 75.44) (width 0.4) (layer F.Cu) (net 27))
 (segment (start 155.121 73.49) (end 151.651 73.49) (width 0.4) (layer F.Cu) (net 27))
 (segment (start 147.921 72.84) (end 151.651 72.84) (width 0.4) (layer F.Cu) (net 27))
 (segment (start 155.121 70.89) (end 153.066 70.89) (width 0.4) (layer F.Cu) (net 27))
 (segment (start 151.651 72.305) (end 151.651 72.84) (width 0.4) (layer F.Cu) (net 27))
 (segment (start 151.651 72.84) (end 151.651 73.49) (width 0.4) (layer F.Cu) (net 27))
 (segment (start 151.651 73.49) (end 151.651 75.44) (width 0.4) (layer F.Cu) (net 27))
 (segment (start 151.651 75.44) (end 151.651 80.775) (width 0.4) (layer F.Cu) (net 27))
 (segment (start 153.066 70.89) (end 151.651 72.305) (width 0.4) (layer F.Cu) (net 27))
 (segment (start 147.921 69.59) (end 145.196 69.59) (width 0.4) (layer F.Cu) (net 28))
 (segment (start 144.921 72.865) (end 144.921 73.825) (width 0.4) (layer F.Cu) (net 28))
 (segment (start 144.761 72.705) (end 144.921 72.865) (width 0.4) (layer F.Cu) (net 28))
 (segment (start 144.761 70.025) (end 144.761 72.705) (width 0.4) (layer F.Cu) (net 28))
 (segment (start 145.196 69.59) (end 144.761 70.025) (width 0.4) (layer F.Cu) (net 28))
 (segment (start 149.451 81.185) (end 149.451 81.405) (width 0.4) (layer F.Cu) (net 29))
 (segment (start 149.451 81.405) (end 150.821 82.775) (width 0.4) (layer F.Cu) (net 29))
 (segment (start 150.821 82.775) (end 151.651 82.775) (width 0.4) (layer F.Cu) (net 29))
 (segment (start 155.121 74.79) (end 153.196 74.79) (width 0.4) (layer F.Cu) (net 29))
 (segment (start 149.451 79.565) (end 149.451 81.185) (width 0.4) (layer F.Cu) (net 29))
 (via (at 149.451 79.565) (size 0.6) (drill 0.4) (layers F.Cu B.Cu) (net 29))
 (segment (start 149.451 77.905) (end 149.451 79.565) (width 0.4) (layer B.Cu) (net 29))
 (segment (start 152.881 74.475) (end 149.451 77.905) (width 0.4) (layer B.Cu) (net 29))
 (via (at 152.881 74.475) (size 0.6) (drill 0.4) (layers F.Cu B.Cu) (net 29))
 (segment (start 153.196 74.79) (end 152.881 74.475) (width 0.4) (layer F.Cu) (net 29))
 (segment (start 144.981 85.345) (end 144.981 87.075) (width 0.4) (layer F.Cu) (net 30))
 (segment (start 157.971 87.075) (end 157.971 85.395) (width 0.4) (layer F.Cu) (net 31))
 (segment (start 150.131 85.155) (end 150.131 86.525) (width 0.4) (layer F.Cu) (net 32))
 (segment (start 149.451 83.565) (end 149.451 84.475) (width 0.5) (layer F.Cu) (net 32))
 (segment (start 150.131 85.155) (end 150.131 85.145) (width 0.4) (layer F.Cu) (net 32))
 (segment (start 149.451 84.475) (end 150.131 85.155) (width 0.4) (layer F.Cu) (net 32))
 (segment (start 147.551 81.185) (end 147.551 81.925) (width 0.5) (layer F.Cu) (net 32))
 (segment (start 147.551 81.925) (end 148.081 82.455) (width 0.5) (layer F.Cu) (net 32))
 (segment (start 148.081 82.455) (end 149.051 82.455) (width 0.5) (layer F.Cu) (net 32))
 (segment (start 149.051 82.455) (end 149.451 82.855) (width 0.5) (layer F.Cu) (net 32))
 (segment (start 149.451 82.855) (end 149.451 83.565) (width 0.5) (layer F.Cu) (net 32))
 (segment (start 144.971 77.905) (end 144.971 78.015) (width 0.4) (layer F.Cu) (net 32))
 (segment (start 144.971 78.015) (end 146.121 79.165) (width 0.5) (layer F.Cu) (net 32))
 (segment (start 146.941 79.165) (end 147.551 79.775) (width 0.5) (layer F.Cu) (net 32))
 (segment (start 146.121 79.165) (end 146.941 79.165) (width 0.5) (layer F.Cu) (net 32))
 (segment (start 147.551 79.835) (end 147.551 81.185) (width 0.4) (layer F.Cu) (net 32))
 (segment (start 155.121 76.09) (end 152.746 76.09) (width 0.4) (layer F.Cu) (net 33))
 (segment (start 158.081 73.495) (end 158.271 73.305) (width 0.5) (layer B.Cu) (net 33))
 (segment (start 158.271 73.305) (end 158.271 72.295) (width 0.5) (layer B.Cu) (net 33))
 (segment (start 158.271 72.295) (end 157.481 71.505) (width 0.5) (layer B.Cu) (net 33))
 (segment (start 157.481 71.505) (end 155.971 71.505) (width 0.5) (layer B.Cu) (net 33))
 (segment (start 155.971 71.505) (end 155.201 72.275) (width 0.5) (layer B.Cu) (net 33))
 (segment (start 155.201 72.275) (end 155.201 75.345) (width 0.5) (layer B.Cu) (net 33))
 (segment (start 155.201 75.345) (end 154.481 76.065) (width 0.5) (layer B.Cu) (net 33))
 (segment (start 154.481 76.065) (end 152.771 76.065) (width 0.5) (layer B.Cu) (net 33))
 (segment (start 152.771 76.065) (end 152.511 76.325) (width 0.5) (layer B.Cu) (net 33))
 (via (at 152.511 76.325) (size 0.6) (drill 0.4) (layers F.Cu B.Cu) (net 33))
 (segment (start 158.081 73.495) (end 158.081 84.335) (width 0.5) (layer B.Cu) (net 33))
 (segment (start 152.746 76.09) (end 152.511 76.325) (width 0.4) (layer F.Cu) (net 33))
 (segment (start 143.821 68.335) (end 143.141 68.335) (width 0.4) (layer F.Cu) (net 19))
 (segment (start 142.6494 67.8434) (end 141.2494 67.8434) (width 0.4) (layer F.Cu) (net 19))
 (segment (start 143.141 68.335) (end 142.6494 67.8434) (width 0.4) (layer F.Cu) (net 19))
 (segment (start 143.811 71.255) (end 143.371 71.255) (width 0.4) (layer F.Cu) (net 20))
 (segment (start 142.4994 70.3834) (end 141.2494 70.3834) (width 0.4) (layer F.Cu) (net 20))
 (segment (start 143.371 71.255) (end 142.4994 70.3834) (width 0.4) (layer F.Cu) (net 20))
 (segment (start 150.781 86.525) (end 150.781 84.335) (width 0.4) (layer F.Cu) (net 48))
 (segment (start 153.326 76.74) (end 152.751 77.315) (width 0.4) (layer F.Cu) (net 48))
 (via (at 152.751 77.315) (size 0.6) (drill 0.4) (layers F.Cu B.Cu) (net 48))
 (segment (start 152.751 77.315) (end 150.781 79.285) (width 0.4) (layer B.Cu) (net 48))
 (segment (start 150.781 79.285) (end 150.781 84.335) (width 0.4) (layer B.Cu) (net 48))
 (via (at 150.781 84.335) (size 0.6) (drill 0.4) (layers F.Cu B.Cu) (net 48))
 (segment (start 153.326 76.74) (end 155.121 76.74) (width 0.4) (layer F.Cu) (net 48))
 (segment (start 151.431 86.525) (end 151.431 85.195) (width 0.4) (layer F.Cu) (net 47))
 (segment (start 151.871 79.505) (end 151.871 83.995) (width 0.4) (layer B.Cu) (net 47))
 (via (at 151.871 83.995) (size 0.6) (drill 0.4) (layers F.Cu B.Cu) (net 47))
 (segment (start 151.871 83.995) (end 151.871 84.755) (width 0.4) (layer F.Cu) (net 47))
 (segment (start 151.871 84.755) (end 151.431 85.195) (width 0.4) (layer F.Cu) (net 47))
 (segment (start 153.986 77.39) (end 155.121 77.39) (width 0.4) (layer F.Cu) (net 47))
 (via (at 153.241 78.135) (size 0.6) (drill 0.4) (layers F.Cu B.Cu) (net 47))
 (segment (start 153.986 77.39) (end 153.241 78.135) (width 0.4) (layer F.Cu) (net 47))
 (segment (start 153.241 78.135) (end 151.871 79.505) (width 0.4) (layer B.Cu) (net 47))
 (segment (start 147.921 68.94) (end 147.056 68.94) (width 0.4) (layer F.Cu) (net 34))
 (segment (start 147.056 68.94) (end 146.451 68.335) (width 0.4) (layer F.Cu) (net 34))
 (segment (start 146.451 68.335) (end 145.721 68.335) (width 0.4) (layer F.Cu) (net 34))
 (segment (start 147.921 71.54) (end 146.666 71.54) (width 0.4) (layer F.Cu) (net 35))
 (segment (start 146.381 71.255) (end 145.711 71.255) (width 0.4) (layer F.Cu) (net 35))
 (segment (start 146.666 71.54) (end 146.381 71.255) (width 0.4) (layer F.Cu) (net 35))
 (segment (start 144.981 83.445) (end 144.981 82.465) (width 0.4) (layer F.Cu) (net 36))
 (segment (start 153.086 72.19) (end 155.121 72.19) (width 0.4) (layer F.Cu) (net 36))
 (segment (start 153.071 72.205) (end 153.086 72.19) (width 0.4) (layer F.Cu) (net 36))
 (via (at 153.071 72.205) (size 0.6) (drill 0.4) (layers F.Cu B.Cu) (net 36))
 (segment (start 147.941 77.335) (end 153.071 72.205) (width 0.4) (layer B.Cu) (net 36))
 (segment (start 147.941 79.505) (end 147.941 77.335) (width 0.4) (layer B.Cu) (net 36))
 (segment (start 144.981 82.465) (end 147.941 79.505) (width 0.4) (layer B.Cu) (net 36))
 (via (at 144.981 82.465) (size 0.6) (drill 0.4) (layers F.Cu B.Cu) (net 36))
 (via (at 157.161 72.865) (size 0.6) (drill 0.4) (layers F.Cu B.Cu) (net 37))
 (segment (start 157.971 83.495) (end 156.221 83.495) (width 0.4) (layer F.Cu) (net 37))
 (segment (start 157.161 82.555) (end 157.161 72.865) (width 0.4) (layer B.Cu) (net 37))
 (segment (start 156.221 83.495) (end 157.161 82.555) (width 0.4) (layer B.Cu) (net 37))
 (via (at 156.221 83.495) (size 0.6) (drill 0.4) (layers F.Cu B.Cu) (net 37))
 (segment (start 157.136 72.84) (end 155.121 72.84) (width 0.4) (layer F.Cu) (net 37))
 (segment (start 157.161 72.865) (end 157.136 72.84) (width 0.4) (layer F.Cu) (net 37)))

